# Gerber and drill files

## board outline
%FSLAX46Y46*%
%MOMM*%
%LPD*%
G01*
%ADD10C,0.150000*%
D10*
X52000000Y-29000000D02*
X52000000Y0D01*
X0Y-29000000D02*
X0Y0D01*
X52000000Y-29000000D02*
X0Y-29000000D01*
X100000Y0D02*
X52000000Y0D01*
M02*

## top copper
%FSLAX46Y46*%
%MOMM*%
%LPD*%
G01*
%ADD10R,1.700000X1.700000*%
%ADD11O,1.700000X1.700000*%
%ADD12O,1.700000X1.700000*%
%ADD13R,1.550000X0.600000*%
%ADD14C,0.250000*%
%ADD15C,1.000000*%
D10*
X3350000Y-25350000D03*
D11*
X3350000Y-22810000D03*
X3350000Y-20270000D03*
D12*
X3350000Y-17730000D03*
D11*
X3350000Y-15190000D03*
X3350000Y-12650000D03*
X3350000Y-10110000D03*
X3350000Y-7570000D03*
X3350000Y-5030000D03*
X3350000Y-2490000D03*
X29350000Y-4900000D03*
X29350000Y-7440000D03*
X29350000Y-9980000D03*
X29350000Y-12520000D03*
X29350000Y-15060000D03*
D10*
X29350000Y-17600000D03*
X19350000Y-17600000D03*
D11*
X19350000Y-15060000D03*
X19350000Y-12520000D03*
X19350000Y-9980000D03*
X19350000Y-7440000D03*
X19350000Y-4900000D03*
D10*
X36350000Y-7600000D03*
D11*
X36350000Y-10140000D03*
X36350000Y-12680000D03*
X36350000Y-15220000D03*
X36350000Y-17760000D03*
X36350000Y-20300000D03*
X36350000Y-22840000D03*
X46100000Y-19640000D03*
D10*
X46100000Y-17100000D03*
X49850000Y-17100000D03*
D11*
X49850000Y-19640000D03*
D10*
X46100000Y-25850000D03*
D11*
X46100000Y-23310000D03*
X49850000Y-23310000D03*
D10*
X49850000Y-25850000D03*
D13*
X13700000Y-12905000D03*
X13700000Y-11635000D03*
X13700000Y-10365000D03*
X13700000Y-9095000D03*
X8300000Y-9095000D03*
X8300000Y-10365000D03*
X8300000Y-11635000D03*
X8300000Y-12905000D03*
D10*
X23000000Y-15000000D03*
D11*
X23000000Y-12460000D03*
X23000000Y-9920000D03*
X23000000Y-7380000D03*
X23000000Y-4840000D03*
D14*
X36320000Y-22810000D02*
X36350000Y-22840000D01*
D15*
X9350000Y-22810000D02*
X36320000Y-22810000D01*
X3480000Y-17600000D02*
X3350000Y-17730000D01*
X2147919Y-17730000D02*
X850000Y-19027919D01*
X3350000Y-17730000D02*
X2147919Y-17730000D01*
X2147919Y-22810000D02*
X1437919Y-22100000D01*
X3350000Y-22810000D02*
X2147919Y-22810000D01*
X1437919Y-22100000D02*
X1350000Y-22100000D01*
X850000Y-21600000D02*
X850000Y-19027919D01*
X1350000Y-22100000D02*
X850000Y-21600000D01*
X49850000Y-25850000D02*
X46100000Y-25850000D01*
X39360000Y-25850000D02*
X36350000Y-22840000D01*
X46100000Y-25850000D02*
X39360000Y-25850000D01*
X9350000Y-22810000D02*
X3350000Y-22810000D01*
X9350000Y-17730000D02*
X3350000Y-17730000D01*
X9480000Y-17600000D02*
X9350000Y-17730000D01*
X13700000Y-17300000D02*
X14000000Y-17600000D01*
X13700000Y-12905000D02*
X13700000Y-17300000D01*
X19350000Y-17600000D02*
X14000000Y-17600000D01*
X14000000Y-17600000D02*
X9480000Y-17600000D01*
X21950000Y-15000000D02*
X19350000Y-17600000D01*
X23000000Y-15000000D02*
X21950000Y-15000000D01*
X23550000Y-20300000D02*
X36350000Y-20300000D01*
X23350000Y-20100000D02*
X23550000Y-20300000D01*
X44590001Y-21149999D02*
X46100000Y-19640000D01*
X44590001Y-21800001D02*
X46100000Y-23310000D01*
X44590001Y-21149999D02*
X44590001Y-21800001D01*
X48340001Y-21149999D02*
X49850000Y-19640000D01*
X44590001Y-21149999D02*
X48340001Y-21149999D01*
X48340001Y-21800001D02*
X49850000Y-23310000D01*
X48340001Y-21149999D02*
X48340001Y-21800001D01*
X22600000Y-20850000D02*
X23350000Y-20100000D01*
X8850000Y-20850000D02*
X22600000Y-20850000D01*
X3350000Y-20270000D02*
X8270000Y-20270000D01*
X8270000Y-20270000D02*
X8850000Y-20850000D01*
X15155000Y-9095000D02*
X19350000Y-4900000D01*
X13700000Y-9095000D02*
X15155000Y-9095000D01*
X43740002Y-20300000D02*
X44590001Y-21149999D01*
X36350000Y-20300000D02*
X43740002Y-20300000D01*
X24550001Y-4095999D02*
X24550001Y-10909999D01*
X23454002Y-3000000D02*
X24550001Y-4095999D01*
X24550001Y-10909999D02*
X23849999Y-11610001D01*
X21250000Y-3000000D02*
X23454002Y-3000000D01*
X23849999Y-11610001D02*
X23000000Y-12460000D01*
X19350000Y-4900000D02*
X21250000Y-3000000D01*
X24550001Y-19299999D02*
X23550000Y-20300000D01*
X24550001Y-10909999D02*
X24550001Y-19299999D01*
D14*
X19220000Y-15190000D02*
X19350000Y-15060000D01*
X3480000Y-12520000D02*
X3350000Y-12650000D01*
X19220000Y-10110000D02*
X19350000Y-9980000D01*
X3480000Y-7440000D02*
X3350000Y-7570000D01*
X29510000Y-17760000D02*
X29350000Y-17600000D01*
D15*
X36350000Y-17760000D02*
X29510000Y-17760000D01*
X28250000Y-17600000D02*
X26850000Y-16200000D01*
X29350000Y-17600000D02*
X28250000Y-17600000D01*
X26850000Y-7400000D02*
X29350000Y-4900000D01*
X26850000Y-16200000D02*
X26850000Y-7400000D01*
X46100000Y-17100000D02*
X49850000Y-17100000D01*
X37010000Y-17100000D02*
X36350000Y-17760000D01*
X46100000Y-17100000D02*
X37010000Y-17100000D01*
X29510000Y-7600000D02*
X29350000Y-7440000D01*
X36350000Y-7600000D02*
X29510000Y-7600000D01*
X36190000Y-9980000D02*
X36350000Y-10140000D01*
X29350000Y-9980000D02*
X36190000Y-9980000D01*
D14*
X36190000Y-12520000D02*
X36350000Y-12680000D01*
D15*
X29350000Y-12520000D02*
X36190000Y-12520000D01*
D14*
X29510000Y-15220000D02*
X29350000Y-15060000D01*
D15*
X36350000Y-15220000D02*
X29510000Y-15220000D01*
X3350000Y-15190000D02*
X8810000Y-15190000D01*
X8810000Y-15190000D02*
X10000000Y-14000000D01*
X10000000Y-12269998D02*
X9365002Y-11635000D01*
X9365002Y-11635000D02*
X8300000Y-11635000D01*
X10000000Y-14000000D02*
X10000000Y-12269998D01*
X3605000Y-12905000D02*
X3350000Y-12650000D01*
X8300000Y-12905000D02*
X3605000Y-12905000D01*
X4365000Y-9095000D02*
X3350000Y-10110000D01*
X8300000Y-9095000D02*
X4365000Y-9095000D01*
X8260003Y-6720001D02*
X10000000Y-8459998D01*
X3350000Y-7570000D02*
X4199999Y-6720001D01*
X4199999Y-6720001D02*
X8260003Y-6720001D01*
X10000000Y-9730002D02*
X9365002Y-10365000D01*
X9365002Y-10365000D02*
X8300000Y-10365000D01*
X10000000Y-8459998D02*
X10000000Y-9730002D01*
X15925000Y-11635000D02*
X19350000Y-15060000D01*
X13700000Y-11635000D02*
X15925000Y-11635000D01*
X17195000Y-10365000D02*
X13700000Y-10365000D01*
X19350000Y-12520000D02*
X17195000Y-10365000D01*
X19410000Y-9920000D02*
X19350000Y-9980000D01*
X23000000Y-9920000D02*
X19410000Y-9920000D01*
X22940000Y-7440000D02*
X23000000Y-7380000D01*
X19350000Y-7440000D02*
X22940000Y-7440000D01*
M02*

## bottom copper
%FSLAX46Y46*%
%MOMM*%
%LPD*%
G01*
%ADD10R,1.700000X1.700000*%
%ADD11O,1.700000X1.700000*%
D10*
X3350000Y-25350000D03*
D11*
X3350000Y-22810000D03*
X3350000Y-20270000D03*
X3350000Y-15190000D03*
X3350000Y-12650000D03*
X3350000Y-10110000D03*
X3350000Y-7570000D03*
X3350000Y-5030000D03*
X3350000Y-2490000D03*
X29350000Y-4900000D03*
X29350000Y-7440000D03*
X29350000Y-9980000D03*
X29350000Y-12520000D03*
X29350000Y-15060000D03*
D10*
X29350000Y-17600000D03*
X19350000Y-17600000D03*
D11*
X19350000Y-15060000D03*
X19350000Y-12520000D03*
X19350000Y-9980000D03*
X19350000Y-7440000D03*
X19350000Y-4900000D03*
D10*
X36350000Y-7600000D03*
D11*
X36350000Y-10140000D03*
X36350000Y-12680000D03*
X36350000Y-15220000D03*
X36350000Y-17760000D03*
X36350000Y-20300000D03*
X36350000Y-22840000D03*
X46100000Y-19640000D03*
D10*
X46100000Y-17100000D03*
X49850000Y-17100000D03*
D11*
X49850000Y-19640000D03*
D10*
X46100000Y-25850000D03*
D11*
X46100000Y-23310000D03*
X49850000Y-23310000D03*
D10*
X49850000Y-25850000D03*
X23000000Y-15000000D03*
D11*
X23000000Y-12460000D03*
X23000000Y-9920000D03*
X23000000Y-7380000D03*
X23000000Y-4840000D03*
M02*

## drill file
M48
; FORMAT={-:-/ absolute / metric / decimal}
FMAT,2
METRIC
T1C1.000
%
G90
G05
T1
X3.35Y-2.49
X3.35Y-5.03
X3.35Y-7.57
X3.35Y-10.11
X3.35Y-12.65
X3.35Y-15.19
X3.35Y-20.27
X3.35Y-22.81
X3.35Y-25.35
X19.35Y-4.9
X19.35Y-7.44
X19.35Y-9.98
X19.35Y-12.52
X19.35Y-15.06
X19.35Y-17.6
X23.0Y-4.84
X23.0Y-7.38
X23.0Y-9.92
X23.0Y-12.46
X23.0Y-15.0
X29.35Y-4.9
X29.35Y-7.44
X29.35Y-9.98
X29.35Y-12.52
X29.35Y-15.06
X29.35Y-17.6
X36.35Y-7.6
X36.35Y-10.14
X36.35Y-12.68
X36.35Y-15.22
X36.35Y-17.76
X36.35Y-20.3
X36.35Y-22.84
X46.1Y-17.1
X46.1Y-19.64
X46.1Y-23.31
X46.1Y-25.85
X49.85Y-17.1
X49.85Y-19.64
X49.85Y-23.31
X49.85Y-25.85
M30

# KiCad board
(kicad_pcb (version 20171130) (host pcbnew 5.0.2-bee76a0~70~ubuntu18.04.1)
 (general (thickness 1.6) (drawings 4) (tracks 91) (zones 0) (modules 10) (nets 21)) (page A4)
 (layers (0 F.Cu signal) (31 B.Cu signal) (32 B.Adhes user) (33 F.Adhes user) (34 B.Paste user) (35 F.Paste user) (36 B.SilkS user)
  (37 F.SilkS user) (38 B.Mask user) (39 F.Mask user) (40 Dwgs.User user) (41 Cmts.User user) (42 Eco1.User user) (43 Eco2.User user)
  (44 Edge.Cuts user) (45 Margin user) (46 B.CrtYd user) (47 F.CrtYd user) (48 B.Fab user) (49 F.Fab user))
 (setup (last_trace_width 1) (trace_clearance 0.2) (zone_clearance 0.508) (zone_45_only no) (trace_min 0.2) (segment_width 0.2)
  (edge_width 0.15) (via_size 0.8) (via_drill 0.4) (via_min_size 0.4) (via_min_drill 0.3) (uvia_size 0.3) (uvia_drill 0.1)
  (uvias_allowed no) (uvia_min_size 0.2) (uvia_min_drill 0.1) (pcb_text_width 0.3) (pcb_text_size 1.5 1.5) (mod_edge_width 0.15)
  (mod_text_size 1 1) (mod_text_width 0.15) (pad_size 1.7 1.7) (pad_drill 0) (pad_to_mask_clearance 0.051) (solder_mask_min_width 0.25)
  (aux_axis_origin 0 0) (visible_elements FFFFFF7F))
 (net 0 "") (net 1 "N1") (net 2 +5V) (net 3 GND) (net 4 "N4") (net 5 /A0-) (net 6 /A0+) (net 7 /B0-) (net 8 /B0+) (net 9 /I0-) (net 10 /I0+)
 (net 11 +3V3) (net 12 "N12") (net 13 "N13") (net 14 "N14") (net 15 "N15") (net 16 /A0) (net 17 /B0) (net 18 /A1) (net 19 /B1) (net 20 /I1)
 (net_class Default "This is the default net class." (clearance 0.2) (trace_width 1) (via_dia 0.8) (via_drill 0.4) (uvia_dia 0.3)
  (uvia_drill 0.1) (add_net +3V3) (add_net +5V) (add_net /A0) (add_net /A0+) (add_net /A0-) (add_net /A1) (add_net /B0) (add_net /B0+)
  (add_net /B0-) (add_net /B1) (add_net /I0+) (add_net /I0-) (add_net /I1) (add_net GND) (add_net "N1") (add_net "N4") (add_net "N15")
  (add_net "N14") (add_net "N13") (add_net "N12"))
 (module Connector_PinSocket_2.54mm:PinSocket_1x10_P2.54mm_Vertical (layer F.Cu) (at 3.35 25.35 180)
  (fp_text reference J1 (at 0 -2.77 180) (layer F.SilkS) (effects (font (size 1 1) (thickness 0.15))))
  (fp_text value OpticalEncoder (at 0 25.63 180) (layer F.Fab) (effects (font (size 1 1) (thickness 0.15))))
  (pad 1 thru_hole rect (at 0 0 180) (size 1.7 1.7) (drill 1) (layers *.Cu *.Mask) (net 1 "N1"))
  (pad 2 thru_hole oval (at 0 2.54 180) (size 1.7 1.7) (drill 1) (layers *.Cu *.Mask) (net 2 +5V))
  (pad 3 thru_hole oval (at 0 5.08 180) (size 1.7 1.7) (drill 1) (layers *.Cu *.Mask) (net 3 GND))
  (pad 4 smd oval (at 0 7.62 180) (size 1.7 1.7) (layers F.Cu F.Paste F.Mask) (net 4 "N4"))
  (pad 5 thru_hole oval (at 0 10.16 180) (size 1.7 1.7) (drill 1) (layers *.Cu *.Mask) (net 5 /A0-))
  (pad 6 thru_hole oval (at 0 12.7 180) (size 1.7 1.7) (drill 1) (layers *.Cu *.Mask) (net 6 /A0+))
  (pad 7 thru_hole oval (at 0 15.24 180) (size 1.7 1.7) (drill 1) (layers *.Cu *.Mask) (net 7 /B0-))
  (pad 8 thru_hole oval (at 0 17.78 180) (size 1.7 1.7) (drill 1) (layers *.Cu *.Mask) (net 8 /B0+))
  (pad 9 thru_hole oval (at 0 20.32 180) (size 1.7 1.7) (drill 1) (layers *.Cu *.Mask) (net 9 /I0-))
  (pad 10 thru_hole oval (at 0 22.86 180) (size 1.7 1.7) (drill 1) (layers *.Cu *.Mask) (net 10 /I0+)))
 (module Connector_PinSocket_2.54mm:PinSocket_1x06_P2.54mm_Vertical (layer F.Cu) (at 29.35 17.6 180)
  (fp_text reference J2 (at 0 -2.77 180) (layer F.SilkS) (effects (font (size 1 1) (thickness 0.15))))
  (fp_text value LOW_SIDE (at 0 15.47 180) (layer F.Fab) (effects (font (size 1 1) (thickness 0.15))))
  (pad 6 thru_hole oval (at 0 12.7 180) (size 1.7 1.7) (drill 1) (layers *.Cu *.Mask) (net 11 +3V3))
  (pad 5 thru_hole oval (at 0 10.16 180) (size 1.7 1.7) (drill 1) (layers *.Cu *.Mask) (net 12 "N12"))
  (pad 4 thru_hole oval (at 0 7.62 180) (size 1.7 1.7) (drill 1) (layers *.Cu *.Mask) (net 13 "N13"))
  (pad 3 thru_hole oval (at 0 5.08 180) (size 1.7 1.7) (drill 1) (layers *.Cu *.Mask) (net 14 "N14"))
  (pad 2 thru_hole oval (at 0 2.54 180) (size 1.7 1.7) (drill 1) (layers *.Cu *.Mask) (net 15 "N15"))
  (pad 1 thru_hole rect (at 0 0 180) (size 1.7 1.7) (drill 1) (layers *.Cu *.Mask) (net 11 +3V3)))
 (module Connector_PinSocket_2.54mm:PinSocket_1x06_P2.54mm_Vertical (layer F.Cu) (at 19.35 17.6 180)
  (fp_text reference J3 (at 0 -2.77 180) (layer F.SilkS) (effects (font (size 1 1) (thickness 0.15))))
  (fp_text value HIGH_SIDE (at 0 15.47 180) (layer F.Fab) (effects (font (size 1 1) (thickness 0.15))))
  (pad 1 thru_hole rect (at 0 0 180) (size 1.7 1.7) (drill 1) (layers *.Cu *.Mask) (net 2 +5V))
  (pad 2 thru_hole oval (at 0 2.54 180) (size 1.7 1.7) (drill 1) (layers *.Cu *.Mask) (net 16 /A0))
  (pad 3 thru_hole oval (at 0 5.08 180) (size 1.7 1.7) (drill 1) (layers *.Cu *.Mask) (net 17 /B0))
  (pad 4 thru_hole oval (at 0 7.62 180) (size 1.7 1.7) (drill 1) (layers *.Cu *.Mask) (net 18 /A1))
  (pad 5 thru_hole oval (at 0 10.16 180) (size 1.7 1.7) (drill 1) (layers *.Cu *.Mask) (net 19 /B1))
  (pad 6 thru_hole oval (at 0 12.7 180) (size 1.7 1.7) (drill 1) (layers *.Cu *.Mask) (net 3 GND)))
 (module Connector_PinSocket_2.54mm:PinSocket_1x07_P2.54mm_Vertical (layer F.Cu) (at 36.35 7.6)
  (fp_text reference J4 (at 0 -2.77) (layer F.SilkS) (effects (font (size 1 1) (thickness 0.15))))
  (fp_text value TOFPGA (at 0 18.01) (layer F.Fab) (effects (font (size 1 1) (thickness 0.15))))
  (pad 1 thru_hole rect (at 0 0) (size 1.7 1.7) (drill 1) (layers *.Cu *.Mask) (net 12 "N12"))
  (pad 2 thru_hole oval (at 0 2.54) (size 1.7 1.7) (drill 1) (layers *.Cu *.Mask) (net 13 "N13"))
  (pad 3 thru_hole oval (at 0 5.08) (size 1.7 1.7) (drill 1) (layers *.Cu *.Mask) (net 14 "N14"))
  (pad 4 thru_hole oval (at 0 7.62) (size 1.7 1.7) (drill 1) (layers *.Cu *.Mask) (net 15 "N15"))
  (pad 5 thru_hole oval (at 0 10.16) (size 1.7 1.7) (drill 1) (layers *.Cu *.Mask) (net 11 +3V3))
  (pad 6 thru_hole oval (at 0 12.7) (size 1.7 1.7) (drill 1) (layers *.Cu *.Mask) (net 3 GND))
  (pad 7 thru_hole oval (at 0 15.24) (size 1.7 1.7) (drill 1) (layers *.Cu *.Mask) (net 2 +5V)))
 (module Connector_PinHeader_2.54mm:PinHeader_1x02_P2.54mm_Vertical (layer F.Cu) (at 46.1 17.1)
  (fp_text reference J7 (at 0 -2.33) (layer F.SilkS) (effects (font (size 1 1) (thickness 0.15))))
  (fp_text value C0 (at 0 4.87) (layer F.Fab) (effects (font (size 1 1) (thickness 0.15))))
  (pad 2 thru_hole oval (at 0 2.54) (size 1.7 1.7) (drill 1) (layers *.Cu *.Mask) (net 3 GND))
  (pad 1 thru_hole rect (at 0 0) (size 1.7 1.7) (drill 1) (layers *.Cu *.Mask) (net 11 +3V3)))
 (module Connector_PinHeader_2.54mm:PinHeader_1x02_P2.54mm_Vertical (layer F.Cu) (at 49.85 17.1)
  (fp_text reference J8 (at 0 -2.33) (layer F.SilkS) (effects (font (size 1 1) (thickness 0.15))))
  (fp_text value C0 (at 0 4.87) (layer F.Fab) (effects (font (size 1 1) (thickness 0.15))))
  (pad 1 thru_hole rect (at 0 0) (size 1.7 1.7) (drill 1) (layers *.Cu *.Mask) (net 11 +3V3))
  (pad 2 thru_hole oval (at 0 2.54) (size 1.7 1.7) (drill 1) (layers *.Cu *.Mask) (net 3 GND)))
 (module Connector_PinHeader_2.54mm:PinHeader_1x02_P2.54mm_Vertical (layer F.Cu) (at 46.1 25.85 180)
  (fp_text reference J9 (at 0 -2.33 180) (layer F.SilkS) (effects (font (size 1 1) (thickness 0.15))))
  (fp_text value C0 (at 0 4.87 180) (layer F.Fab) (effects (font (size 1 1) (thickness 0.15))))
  (pad 1 thru_hole rect (at 0 0 180) (size 1.7 1.7) (drill 1) (layers *.Cu *.Mask) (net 2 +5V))
  (pad 2 thru_hole oval (at 0 2.54 180) (size 1.7 1.7) (drill 1) (layers *.Cu *.Mask) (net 3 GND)))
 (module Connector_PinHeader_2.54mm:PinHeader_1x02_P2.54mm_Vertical (layer F.Cu) (at 49.85 25.85 180)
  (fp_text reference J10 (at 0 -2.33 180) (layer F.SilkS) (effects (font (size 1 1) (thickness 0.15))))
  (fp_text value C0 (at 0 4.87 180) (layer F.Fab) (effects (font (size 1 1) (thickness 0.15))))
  (pad 2 thru_hole oval (at 0 2.54 180) (size 1.7 1.7) (drill 1) (layers *.Cu *.Mask) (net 3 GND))
  (pad 1 thru_hole rect (at 0 0 180) (size 1.7 1.7) (drill 1) (layers *.Cu *.Mask) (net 2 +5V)))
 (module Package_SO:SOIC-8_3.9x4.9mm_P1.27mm (layer F.Cu) (at 11 11 180)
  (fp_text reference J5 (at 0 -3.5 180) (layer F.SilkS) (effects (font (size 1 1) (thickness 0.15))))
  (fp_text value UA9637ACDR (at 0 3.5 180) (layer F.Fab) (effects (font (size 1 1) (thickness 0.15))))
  (pad 1 smd rect (at -2.7 -1.905 180) (size 1.55 0.6) (layers F.Cu F.Paste F.Mask) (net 2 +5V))
  (pad 2 smd rect (at -2.7 -0.635 180) (size 1.55 0.6) (layers F.Cu F.Paste F.Mask) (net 16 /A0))
  (pad 3 smd rect (at -2.7 0.635 180) (size 1.55 0.6) (layers F.Cu F.Paste F.Mask) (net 17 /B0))
  (pad 4 smd rect (at -2.7 1.905 180) (size 1.55 0.6) (layers F.Cu F.Paste F.Mask) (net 3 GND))
  (pad 5 smd rect (at 2.7 1.905 180) (size 1.55 0.6) (layers F.Cu F.Paste F.Mask) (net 7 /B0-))
  (pad 6 smd rect (at 2.7 0.635 180) (size 1.55 0.6) (layers F.Cu F.Paste F.Mask) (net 8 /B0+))
  (pad 7 smd rect (at 2.7 -0.635 180) (size 1.55 0.6) (layers F.Cu F.Paste F.Mask) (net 5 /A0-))
  (pad 8 smd rect (at 2.7 -1.905 180) (size 1.55 0.6) (layers F.Cu F.Paste F.Mask) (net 6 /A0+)))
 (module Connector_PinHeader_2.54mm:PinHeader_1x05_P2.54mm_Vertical (layer F.Cu) (at 23 15 180)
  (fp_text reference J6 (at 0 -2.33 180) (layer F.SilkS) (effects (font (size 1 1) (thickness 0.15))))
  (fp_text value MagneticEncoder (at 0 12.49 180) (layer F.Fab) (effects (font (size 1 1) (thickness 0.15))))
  (pad 1 thru_hole rect (at 0 0 180) (size 1.7 1.7) (drill 1) (layers *.Cu *.Mask) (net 2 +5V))
  (pad 2 thru_hole oval (at 0 2.54 180) (size 1.7 1.7) (drill 1) (layers *.Cu *.Mask) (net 3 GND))
  (pad 3 thru_hole oval (at 0 5.08 180) (size 1.7 1.7) (drill 1) (layers *.Cu *.Mask) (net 18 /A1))
  (pad 4 thru_hole oval (at 0 7.62 180) (size 1.7 1.7) (drill 1) (layers *.Cu *.Mask) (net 19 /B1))
  (pad 5 thru_hole oval (at 0 10.16 180) (size 1.7 1.7) (drill 1) (layers *.Cu *.Mask) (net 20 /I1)))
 (gr_line (start 52 29) (end 52 0) (layer Edge.Cuts) (width 0.15))
 (gr_line (start 0 29) (end 0 0) (layer Edge.Cuts) (width 0.15))
 (gr_line (start 52 29) (end 0 29) (layer Edge.Cuts) (width 0.15))
 (gr_line (start 0.1 0) (end 52 0) (layer Edge.Cuts) (width 0.15))
 (segment (start 36.32 22.81) (end 36.35 22.84) (width 0.25) (layer F.Cu) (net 2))
 (segment (start 9.35 22.81) (end 36.32 22.81) (width 1) (layer F.Cu) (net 2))
 (segment (start 3.48 17.6) (end 3.35 17.73) (width 1) (layer F.Cu) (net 2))
 (segment (start 2.147919 17.73) (end 0.85 19.027919) (width 1) (layer F.Cu) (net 2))
 (segment (start 3.35 17.73) (end 2.147919 17.73) (width 1) (layer F.Cu) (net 2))
 (segment (start 2.147919 22.81) (end 1.437919 22.1) (width 1) (layer F.Cu) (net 2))
 (segment (start 3.35 22.81) (end 2.147919 22.81) (width 1) (layer F.Cu) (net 2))
 (segment (start 1.437919 22.1) (end 1.35 22.1) (width 1) (layer F.Cu) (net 2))
 (segment (start 0.85 21.6) (end 0.85 19.027919) (width 1) (layer F.Cu) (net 2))
 (segment (start 1.35 22.1) (end 0.85 21.6) (width 1) (layer F.Cu) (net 2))
 (segment (start 49.85 25.85) (end 46.1 25.85) (width 1) (layer F.Cu) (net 2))
 (segment (start 39.36 25.85) (end 36.35 22.84) (width 1) (layer F.Cu) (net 2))
 (segment (start 46.1 25.85) (end 39.36 25.85) (width 1) (layer F.Cu) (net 2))
 (segment (start 9.35 22.81) (end 3.35 22.81) (width 1) (layer F.Cu) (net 2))
 (segment (start 9.35 17.73) (end 3.35 17.73) (width 1) (layer F.Cu) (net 2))
 (segment (start 9.48 17.6) (end 9.35 17.73) (width 1) (layer F.Cu) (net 2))
 (segment (start 13.7 17.3) (end 14 17.6) (width 1) (layer F.Cu) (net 2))
 (segment (start 13.7 12.905) (end 13.7 17.3) (width 1) (layer F.Cu) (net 2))
 (segment (start 19.35 17.6) (end 14 17.6) (width 1) (layer F.Cu) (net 2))
 (segment (start 14 17.6) (end 9.48 17.6) (width 1) (layer F.Cu) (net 2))
 (segment (start 21.95 15) (end 19.35 17.6) (width 1) (layer F.Cu) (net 2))
 (segment (start 23 15) (end 21.95 15) (width 1) (layer F.Cu) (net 2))
 (segment (start 23.55 20.3) (end 36.35 20.3) (width 1) (layer F.Cu) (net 3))
 (segment (start 23.35 20.1) (end 23.55 20.3) (width 1) (layer F.Cu) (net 3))
 (segment (start 44.590001 21.149999) (end 46.1 19.64) (width 1) (layer F.Cu) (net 3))
 (segment (start 44.590001 21.800001) (end 46.1 23.31) (width 1) (layer F.Cu) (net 3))
 (segment (start 44.590001 21.149999) (end 44.590001 21.800001) (width 1) (layer F.Cu) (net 3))
 (segment (start 48.340001 21.149999) (end 49.85 19.64) (width 1) (layer F.Cu) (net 3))
 (segment (start 44.590001 21.149999) (end 48.340001 21.149999) (width 1) (layer F.Cu) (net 3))
 (segment (start 48.340001 21.800001) (end 49.85 23.31) (width 1) (layer F.Cu) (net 3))
 (segment (start 48.340001 21.149999) (end 48.340001 21.800001) (width 1) (layer F.Cu) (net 3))
 (segment (start 22.6 20.85) (end 23.35 20.1) (width 1) (layer F.Cu) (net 3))
 (segment (start 8.85 20.85) (end 22.6 20.85) (width 1) (layer F.Cu) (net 3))
 (segment (start 3.35 20.27) (end 8.27 20.27) (width 1) (layer F.Cu) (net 3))
 (segment (start 8.27 20.27) (end 8.85 20.85) (width 1) (layer F.Cu) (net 3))
 (segment (start 15.155 9.095) (end 19.35 4.9) (width 1) (layer F.Cu) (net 3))
 (segment (start 13.7 9.095) (end 15.155 9.095) (width 1) (layer F.Cu) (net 3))
 (segment (start 43.740002 20.3) (end 44.590001 21.149999) (width 1) (layer F.Cu) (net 3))
 (segment (start 36.35 20.3) (end 43.740002 20.3) (width 1) (layer F.Cu) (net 3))
 (segment (start 24.550001 4.095999) (end 24.550001 10.909999) (width 1) (layer F.Cu) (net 3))
 (segment (start 23.454002 3) (end 24.550001 4.095999) (width 1) (layer F.Cu) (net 3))
 (segment (start 24.550001 10.909999) (end 23.849999 11.610001) (width 1) (layer F.Cu) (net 3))
 (segment (start 21.25 3) (end 23.454002 3) (width 1) (layer F.Cu) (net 3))
 (segment (start 23.849999 11.610001) (end 23 12.46) (width 1) (layer F.Cu) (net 3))
 (segment (start 19.35 4.9) (end 21.25 3) (width 1) (layer F.Cu) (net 3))
 (segment (start 24.550001 19.299999) (end 23.55 20.3) (width 1) (layer F.Cu) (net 3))
 (segment (start 24.550001 10.909999) (end 24.550001 19.299999) (width 1) (layer F.Cu) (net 3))
 (segment (start 19.22 15.19) (end 19.35 15.06) (width 0.25) (layer F.Cu) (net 16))
 (segment (start 3.48 12.52) (end 3.35 12.65) (width 0.25) (layer F.Cu) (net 6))
 (segment (start 19.22 10.11) (end 19.35 9.98) (width 0.25) (layer F.Cu) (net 18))
 (segment (start 3.48 7.44) (end 3.35 7.57) (width 0.25) (layer F.Cu) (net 8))
 (segment (start 29.51 17.76) (end 29.35 17.6) (width 0.25) (layer F.Cu) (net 11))
 (segment (start 36.35 17.76) (end 29.51 17.76) (width 1) (layer F.Cu) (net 11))
 (segment (start 28.25 17.6) (end 26.85 16.2) (width 1) (layer F.Cu) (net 11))
 (segment (start 29.35 17.6) (end 28.25 17.6) (width 1) (layer F.Cu) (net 11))
 (segment (start 26.85 7.4) (end 29.35 4.9) (width 1) (layer F.Cu) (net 11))
 (segment (start 26.85 16.2) (end 26.85 7.4) (width 1) (layer F.Cu) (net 11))
 (segment (start 46.1 17.1) (end 49.85 17.1) (width 1) (layer F.Cu) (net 11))
 (segment (start 37.01 17.1) (end 36.35 17.76) (width 1) (layer F.Cu) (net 11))
 (segment (start 46.1 17.1) (end 37.01 17.1) (width 1) (layer F.Cu) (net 11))
 (segment (start 29.51 7.6) (end 29.35 7.44) (width 1) (layer F.Cu) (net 12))
 (segment (start 36.35 7.6) (end 29.51 7.6) (width 1) (layer F.Cu) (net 12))
 (segment (start 36.19 9.98) (end 36.35 10.14) (width 1) (layer F.Cu) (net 13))
 (segment (start 29.35 9.98) (end 36.19 9.98) (width 1) (layer F.Cu) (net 13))
 (segment (start 36.19 12.52) (end 36.35 12.68) (width 0.25) (layer F.Cu) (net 14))
 (segment (start 29.35 12.52) (end 36.19 12.52) (width 1) (layer F.Cu) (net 14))
 (segment (start 29.51 15.22) (end 29.35 15.06) (width 0.25) (layer F.Cu) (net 15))
 (segment (start 36.35 15.22) (end 29.51 15.22) (width 1) (layer F.Cu) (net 15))
 (segment (start 3.35 15.19) (end 8.81 15.19) (width 1) (layer F.Cu) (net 5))
 (segment (start 8.81 15.19) (end 10 14) (width 1) (layer F.Cu) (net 5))
 (segment (start 10 12.269998) (end 9.365002 11.635) (width 1) (layer F.Cu) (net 5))
 (segment (start 9.365002 11.635) (end 8.3 11.635) (width 1) (layer F.Cu) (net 5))
 (segment (start 10 14) (end 10 12.269998) (width 1) (layer F.Cu) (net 5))
 (segment (start 3.605 12.905) (end 3.35 12.65) (width 1) (layer F.Cu) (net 6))
 (segment (start 8.3 12.905) (end 3.605 12.905) (width 1) (layer F.Cu) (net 6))
 (segment (start 4.365 9.095) (end 3.35 10.11) (width 1) (layer F.Cu) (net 7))
 (segment (start 8.3 9.095) (end 4.365 9.095) (width 1) (layer F.Cu) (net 7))
 (segment (start 8.260003 6.720001) (end 10 8.459998) (width 1) (layer F.Cu) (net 8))
 (segment (start 3.35 7.57) (end 4.199999 6.720001) (width 1) (layer F.Cu) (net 8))
 (segment (start 4.199999 6.720001) (end 8.260003 6.720001) (width 1) (layer F.Cu) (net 8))
 (segment (start 10 9.730002) (end 9.365002 10.365) (width 1) (layer F.Cu) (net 8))
 (segment (start 9.365002 10.365) (end 8.3 10.365) (width 1) (layer F.Cu) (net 8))
 (segment (start 10 8.459998) (end 10 9.730002) (width 1) (layer F.Cu) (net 8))
 (segment (start 15.925 11.635) (end 19.35 15.06) (width 1) (layer F.Cu) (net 16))
 (segment (start 13.7 11.635) (end 15.925 11.635) (width 1) (layer F.Cu) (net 16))
 (segment (start 17.195 10.365) (end 13.7 10.365) (width 1) (layer F.Cu) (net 17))
 (segment (start 19.35 12.52) (end 17.195 10.365) (width 1) (layer F.Cu) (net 17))
 (segment (start 19.41 9.92) (end 19.35 9.98) (width 1) (layer F.Cu) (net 18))
 (segment (start 23 9.92) (end 19.41 9.92) (width 1) (layer F.Cu) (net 18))
 (segment (start 22.94 7.44) (end 23 7.38) (width 1) (layer F.Cu) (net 19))
 (segment (start 19.35 7.44) (end 22.94 7.44) (width 1) (layer F.Cu) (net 19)))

